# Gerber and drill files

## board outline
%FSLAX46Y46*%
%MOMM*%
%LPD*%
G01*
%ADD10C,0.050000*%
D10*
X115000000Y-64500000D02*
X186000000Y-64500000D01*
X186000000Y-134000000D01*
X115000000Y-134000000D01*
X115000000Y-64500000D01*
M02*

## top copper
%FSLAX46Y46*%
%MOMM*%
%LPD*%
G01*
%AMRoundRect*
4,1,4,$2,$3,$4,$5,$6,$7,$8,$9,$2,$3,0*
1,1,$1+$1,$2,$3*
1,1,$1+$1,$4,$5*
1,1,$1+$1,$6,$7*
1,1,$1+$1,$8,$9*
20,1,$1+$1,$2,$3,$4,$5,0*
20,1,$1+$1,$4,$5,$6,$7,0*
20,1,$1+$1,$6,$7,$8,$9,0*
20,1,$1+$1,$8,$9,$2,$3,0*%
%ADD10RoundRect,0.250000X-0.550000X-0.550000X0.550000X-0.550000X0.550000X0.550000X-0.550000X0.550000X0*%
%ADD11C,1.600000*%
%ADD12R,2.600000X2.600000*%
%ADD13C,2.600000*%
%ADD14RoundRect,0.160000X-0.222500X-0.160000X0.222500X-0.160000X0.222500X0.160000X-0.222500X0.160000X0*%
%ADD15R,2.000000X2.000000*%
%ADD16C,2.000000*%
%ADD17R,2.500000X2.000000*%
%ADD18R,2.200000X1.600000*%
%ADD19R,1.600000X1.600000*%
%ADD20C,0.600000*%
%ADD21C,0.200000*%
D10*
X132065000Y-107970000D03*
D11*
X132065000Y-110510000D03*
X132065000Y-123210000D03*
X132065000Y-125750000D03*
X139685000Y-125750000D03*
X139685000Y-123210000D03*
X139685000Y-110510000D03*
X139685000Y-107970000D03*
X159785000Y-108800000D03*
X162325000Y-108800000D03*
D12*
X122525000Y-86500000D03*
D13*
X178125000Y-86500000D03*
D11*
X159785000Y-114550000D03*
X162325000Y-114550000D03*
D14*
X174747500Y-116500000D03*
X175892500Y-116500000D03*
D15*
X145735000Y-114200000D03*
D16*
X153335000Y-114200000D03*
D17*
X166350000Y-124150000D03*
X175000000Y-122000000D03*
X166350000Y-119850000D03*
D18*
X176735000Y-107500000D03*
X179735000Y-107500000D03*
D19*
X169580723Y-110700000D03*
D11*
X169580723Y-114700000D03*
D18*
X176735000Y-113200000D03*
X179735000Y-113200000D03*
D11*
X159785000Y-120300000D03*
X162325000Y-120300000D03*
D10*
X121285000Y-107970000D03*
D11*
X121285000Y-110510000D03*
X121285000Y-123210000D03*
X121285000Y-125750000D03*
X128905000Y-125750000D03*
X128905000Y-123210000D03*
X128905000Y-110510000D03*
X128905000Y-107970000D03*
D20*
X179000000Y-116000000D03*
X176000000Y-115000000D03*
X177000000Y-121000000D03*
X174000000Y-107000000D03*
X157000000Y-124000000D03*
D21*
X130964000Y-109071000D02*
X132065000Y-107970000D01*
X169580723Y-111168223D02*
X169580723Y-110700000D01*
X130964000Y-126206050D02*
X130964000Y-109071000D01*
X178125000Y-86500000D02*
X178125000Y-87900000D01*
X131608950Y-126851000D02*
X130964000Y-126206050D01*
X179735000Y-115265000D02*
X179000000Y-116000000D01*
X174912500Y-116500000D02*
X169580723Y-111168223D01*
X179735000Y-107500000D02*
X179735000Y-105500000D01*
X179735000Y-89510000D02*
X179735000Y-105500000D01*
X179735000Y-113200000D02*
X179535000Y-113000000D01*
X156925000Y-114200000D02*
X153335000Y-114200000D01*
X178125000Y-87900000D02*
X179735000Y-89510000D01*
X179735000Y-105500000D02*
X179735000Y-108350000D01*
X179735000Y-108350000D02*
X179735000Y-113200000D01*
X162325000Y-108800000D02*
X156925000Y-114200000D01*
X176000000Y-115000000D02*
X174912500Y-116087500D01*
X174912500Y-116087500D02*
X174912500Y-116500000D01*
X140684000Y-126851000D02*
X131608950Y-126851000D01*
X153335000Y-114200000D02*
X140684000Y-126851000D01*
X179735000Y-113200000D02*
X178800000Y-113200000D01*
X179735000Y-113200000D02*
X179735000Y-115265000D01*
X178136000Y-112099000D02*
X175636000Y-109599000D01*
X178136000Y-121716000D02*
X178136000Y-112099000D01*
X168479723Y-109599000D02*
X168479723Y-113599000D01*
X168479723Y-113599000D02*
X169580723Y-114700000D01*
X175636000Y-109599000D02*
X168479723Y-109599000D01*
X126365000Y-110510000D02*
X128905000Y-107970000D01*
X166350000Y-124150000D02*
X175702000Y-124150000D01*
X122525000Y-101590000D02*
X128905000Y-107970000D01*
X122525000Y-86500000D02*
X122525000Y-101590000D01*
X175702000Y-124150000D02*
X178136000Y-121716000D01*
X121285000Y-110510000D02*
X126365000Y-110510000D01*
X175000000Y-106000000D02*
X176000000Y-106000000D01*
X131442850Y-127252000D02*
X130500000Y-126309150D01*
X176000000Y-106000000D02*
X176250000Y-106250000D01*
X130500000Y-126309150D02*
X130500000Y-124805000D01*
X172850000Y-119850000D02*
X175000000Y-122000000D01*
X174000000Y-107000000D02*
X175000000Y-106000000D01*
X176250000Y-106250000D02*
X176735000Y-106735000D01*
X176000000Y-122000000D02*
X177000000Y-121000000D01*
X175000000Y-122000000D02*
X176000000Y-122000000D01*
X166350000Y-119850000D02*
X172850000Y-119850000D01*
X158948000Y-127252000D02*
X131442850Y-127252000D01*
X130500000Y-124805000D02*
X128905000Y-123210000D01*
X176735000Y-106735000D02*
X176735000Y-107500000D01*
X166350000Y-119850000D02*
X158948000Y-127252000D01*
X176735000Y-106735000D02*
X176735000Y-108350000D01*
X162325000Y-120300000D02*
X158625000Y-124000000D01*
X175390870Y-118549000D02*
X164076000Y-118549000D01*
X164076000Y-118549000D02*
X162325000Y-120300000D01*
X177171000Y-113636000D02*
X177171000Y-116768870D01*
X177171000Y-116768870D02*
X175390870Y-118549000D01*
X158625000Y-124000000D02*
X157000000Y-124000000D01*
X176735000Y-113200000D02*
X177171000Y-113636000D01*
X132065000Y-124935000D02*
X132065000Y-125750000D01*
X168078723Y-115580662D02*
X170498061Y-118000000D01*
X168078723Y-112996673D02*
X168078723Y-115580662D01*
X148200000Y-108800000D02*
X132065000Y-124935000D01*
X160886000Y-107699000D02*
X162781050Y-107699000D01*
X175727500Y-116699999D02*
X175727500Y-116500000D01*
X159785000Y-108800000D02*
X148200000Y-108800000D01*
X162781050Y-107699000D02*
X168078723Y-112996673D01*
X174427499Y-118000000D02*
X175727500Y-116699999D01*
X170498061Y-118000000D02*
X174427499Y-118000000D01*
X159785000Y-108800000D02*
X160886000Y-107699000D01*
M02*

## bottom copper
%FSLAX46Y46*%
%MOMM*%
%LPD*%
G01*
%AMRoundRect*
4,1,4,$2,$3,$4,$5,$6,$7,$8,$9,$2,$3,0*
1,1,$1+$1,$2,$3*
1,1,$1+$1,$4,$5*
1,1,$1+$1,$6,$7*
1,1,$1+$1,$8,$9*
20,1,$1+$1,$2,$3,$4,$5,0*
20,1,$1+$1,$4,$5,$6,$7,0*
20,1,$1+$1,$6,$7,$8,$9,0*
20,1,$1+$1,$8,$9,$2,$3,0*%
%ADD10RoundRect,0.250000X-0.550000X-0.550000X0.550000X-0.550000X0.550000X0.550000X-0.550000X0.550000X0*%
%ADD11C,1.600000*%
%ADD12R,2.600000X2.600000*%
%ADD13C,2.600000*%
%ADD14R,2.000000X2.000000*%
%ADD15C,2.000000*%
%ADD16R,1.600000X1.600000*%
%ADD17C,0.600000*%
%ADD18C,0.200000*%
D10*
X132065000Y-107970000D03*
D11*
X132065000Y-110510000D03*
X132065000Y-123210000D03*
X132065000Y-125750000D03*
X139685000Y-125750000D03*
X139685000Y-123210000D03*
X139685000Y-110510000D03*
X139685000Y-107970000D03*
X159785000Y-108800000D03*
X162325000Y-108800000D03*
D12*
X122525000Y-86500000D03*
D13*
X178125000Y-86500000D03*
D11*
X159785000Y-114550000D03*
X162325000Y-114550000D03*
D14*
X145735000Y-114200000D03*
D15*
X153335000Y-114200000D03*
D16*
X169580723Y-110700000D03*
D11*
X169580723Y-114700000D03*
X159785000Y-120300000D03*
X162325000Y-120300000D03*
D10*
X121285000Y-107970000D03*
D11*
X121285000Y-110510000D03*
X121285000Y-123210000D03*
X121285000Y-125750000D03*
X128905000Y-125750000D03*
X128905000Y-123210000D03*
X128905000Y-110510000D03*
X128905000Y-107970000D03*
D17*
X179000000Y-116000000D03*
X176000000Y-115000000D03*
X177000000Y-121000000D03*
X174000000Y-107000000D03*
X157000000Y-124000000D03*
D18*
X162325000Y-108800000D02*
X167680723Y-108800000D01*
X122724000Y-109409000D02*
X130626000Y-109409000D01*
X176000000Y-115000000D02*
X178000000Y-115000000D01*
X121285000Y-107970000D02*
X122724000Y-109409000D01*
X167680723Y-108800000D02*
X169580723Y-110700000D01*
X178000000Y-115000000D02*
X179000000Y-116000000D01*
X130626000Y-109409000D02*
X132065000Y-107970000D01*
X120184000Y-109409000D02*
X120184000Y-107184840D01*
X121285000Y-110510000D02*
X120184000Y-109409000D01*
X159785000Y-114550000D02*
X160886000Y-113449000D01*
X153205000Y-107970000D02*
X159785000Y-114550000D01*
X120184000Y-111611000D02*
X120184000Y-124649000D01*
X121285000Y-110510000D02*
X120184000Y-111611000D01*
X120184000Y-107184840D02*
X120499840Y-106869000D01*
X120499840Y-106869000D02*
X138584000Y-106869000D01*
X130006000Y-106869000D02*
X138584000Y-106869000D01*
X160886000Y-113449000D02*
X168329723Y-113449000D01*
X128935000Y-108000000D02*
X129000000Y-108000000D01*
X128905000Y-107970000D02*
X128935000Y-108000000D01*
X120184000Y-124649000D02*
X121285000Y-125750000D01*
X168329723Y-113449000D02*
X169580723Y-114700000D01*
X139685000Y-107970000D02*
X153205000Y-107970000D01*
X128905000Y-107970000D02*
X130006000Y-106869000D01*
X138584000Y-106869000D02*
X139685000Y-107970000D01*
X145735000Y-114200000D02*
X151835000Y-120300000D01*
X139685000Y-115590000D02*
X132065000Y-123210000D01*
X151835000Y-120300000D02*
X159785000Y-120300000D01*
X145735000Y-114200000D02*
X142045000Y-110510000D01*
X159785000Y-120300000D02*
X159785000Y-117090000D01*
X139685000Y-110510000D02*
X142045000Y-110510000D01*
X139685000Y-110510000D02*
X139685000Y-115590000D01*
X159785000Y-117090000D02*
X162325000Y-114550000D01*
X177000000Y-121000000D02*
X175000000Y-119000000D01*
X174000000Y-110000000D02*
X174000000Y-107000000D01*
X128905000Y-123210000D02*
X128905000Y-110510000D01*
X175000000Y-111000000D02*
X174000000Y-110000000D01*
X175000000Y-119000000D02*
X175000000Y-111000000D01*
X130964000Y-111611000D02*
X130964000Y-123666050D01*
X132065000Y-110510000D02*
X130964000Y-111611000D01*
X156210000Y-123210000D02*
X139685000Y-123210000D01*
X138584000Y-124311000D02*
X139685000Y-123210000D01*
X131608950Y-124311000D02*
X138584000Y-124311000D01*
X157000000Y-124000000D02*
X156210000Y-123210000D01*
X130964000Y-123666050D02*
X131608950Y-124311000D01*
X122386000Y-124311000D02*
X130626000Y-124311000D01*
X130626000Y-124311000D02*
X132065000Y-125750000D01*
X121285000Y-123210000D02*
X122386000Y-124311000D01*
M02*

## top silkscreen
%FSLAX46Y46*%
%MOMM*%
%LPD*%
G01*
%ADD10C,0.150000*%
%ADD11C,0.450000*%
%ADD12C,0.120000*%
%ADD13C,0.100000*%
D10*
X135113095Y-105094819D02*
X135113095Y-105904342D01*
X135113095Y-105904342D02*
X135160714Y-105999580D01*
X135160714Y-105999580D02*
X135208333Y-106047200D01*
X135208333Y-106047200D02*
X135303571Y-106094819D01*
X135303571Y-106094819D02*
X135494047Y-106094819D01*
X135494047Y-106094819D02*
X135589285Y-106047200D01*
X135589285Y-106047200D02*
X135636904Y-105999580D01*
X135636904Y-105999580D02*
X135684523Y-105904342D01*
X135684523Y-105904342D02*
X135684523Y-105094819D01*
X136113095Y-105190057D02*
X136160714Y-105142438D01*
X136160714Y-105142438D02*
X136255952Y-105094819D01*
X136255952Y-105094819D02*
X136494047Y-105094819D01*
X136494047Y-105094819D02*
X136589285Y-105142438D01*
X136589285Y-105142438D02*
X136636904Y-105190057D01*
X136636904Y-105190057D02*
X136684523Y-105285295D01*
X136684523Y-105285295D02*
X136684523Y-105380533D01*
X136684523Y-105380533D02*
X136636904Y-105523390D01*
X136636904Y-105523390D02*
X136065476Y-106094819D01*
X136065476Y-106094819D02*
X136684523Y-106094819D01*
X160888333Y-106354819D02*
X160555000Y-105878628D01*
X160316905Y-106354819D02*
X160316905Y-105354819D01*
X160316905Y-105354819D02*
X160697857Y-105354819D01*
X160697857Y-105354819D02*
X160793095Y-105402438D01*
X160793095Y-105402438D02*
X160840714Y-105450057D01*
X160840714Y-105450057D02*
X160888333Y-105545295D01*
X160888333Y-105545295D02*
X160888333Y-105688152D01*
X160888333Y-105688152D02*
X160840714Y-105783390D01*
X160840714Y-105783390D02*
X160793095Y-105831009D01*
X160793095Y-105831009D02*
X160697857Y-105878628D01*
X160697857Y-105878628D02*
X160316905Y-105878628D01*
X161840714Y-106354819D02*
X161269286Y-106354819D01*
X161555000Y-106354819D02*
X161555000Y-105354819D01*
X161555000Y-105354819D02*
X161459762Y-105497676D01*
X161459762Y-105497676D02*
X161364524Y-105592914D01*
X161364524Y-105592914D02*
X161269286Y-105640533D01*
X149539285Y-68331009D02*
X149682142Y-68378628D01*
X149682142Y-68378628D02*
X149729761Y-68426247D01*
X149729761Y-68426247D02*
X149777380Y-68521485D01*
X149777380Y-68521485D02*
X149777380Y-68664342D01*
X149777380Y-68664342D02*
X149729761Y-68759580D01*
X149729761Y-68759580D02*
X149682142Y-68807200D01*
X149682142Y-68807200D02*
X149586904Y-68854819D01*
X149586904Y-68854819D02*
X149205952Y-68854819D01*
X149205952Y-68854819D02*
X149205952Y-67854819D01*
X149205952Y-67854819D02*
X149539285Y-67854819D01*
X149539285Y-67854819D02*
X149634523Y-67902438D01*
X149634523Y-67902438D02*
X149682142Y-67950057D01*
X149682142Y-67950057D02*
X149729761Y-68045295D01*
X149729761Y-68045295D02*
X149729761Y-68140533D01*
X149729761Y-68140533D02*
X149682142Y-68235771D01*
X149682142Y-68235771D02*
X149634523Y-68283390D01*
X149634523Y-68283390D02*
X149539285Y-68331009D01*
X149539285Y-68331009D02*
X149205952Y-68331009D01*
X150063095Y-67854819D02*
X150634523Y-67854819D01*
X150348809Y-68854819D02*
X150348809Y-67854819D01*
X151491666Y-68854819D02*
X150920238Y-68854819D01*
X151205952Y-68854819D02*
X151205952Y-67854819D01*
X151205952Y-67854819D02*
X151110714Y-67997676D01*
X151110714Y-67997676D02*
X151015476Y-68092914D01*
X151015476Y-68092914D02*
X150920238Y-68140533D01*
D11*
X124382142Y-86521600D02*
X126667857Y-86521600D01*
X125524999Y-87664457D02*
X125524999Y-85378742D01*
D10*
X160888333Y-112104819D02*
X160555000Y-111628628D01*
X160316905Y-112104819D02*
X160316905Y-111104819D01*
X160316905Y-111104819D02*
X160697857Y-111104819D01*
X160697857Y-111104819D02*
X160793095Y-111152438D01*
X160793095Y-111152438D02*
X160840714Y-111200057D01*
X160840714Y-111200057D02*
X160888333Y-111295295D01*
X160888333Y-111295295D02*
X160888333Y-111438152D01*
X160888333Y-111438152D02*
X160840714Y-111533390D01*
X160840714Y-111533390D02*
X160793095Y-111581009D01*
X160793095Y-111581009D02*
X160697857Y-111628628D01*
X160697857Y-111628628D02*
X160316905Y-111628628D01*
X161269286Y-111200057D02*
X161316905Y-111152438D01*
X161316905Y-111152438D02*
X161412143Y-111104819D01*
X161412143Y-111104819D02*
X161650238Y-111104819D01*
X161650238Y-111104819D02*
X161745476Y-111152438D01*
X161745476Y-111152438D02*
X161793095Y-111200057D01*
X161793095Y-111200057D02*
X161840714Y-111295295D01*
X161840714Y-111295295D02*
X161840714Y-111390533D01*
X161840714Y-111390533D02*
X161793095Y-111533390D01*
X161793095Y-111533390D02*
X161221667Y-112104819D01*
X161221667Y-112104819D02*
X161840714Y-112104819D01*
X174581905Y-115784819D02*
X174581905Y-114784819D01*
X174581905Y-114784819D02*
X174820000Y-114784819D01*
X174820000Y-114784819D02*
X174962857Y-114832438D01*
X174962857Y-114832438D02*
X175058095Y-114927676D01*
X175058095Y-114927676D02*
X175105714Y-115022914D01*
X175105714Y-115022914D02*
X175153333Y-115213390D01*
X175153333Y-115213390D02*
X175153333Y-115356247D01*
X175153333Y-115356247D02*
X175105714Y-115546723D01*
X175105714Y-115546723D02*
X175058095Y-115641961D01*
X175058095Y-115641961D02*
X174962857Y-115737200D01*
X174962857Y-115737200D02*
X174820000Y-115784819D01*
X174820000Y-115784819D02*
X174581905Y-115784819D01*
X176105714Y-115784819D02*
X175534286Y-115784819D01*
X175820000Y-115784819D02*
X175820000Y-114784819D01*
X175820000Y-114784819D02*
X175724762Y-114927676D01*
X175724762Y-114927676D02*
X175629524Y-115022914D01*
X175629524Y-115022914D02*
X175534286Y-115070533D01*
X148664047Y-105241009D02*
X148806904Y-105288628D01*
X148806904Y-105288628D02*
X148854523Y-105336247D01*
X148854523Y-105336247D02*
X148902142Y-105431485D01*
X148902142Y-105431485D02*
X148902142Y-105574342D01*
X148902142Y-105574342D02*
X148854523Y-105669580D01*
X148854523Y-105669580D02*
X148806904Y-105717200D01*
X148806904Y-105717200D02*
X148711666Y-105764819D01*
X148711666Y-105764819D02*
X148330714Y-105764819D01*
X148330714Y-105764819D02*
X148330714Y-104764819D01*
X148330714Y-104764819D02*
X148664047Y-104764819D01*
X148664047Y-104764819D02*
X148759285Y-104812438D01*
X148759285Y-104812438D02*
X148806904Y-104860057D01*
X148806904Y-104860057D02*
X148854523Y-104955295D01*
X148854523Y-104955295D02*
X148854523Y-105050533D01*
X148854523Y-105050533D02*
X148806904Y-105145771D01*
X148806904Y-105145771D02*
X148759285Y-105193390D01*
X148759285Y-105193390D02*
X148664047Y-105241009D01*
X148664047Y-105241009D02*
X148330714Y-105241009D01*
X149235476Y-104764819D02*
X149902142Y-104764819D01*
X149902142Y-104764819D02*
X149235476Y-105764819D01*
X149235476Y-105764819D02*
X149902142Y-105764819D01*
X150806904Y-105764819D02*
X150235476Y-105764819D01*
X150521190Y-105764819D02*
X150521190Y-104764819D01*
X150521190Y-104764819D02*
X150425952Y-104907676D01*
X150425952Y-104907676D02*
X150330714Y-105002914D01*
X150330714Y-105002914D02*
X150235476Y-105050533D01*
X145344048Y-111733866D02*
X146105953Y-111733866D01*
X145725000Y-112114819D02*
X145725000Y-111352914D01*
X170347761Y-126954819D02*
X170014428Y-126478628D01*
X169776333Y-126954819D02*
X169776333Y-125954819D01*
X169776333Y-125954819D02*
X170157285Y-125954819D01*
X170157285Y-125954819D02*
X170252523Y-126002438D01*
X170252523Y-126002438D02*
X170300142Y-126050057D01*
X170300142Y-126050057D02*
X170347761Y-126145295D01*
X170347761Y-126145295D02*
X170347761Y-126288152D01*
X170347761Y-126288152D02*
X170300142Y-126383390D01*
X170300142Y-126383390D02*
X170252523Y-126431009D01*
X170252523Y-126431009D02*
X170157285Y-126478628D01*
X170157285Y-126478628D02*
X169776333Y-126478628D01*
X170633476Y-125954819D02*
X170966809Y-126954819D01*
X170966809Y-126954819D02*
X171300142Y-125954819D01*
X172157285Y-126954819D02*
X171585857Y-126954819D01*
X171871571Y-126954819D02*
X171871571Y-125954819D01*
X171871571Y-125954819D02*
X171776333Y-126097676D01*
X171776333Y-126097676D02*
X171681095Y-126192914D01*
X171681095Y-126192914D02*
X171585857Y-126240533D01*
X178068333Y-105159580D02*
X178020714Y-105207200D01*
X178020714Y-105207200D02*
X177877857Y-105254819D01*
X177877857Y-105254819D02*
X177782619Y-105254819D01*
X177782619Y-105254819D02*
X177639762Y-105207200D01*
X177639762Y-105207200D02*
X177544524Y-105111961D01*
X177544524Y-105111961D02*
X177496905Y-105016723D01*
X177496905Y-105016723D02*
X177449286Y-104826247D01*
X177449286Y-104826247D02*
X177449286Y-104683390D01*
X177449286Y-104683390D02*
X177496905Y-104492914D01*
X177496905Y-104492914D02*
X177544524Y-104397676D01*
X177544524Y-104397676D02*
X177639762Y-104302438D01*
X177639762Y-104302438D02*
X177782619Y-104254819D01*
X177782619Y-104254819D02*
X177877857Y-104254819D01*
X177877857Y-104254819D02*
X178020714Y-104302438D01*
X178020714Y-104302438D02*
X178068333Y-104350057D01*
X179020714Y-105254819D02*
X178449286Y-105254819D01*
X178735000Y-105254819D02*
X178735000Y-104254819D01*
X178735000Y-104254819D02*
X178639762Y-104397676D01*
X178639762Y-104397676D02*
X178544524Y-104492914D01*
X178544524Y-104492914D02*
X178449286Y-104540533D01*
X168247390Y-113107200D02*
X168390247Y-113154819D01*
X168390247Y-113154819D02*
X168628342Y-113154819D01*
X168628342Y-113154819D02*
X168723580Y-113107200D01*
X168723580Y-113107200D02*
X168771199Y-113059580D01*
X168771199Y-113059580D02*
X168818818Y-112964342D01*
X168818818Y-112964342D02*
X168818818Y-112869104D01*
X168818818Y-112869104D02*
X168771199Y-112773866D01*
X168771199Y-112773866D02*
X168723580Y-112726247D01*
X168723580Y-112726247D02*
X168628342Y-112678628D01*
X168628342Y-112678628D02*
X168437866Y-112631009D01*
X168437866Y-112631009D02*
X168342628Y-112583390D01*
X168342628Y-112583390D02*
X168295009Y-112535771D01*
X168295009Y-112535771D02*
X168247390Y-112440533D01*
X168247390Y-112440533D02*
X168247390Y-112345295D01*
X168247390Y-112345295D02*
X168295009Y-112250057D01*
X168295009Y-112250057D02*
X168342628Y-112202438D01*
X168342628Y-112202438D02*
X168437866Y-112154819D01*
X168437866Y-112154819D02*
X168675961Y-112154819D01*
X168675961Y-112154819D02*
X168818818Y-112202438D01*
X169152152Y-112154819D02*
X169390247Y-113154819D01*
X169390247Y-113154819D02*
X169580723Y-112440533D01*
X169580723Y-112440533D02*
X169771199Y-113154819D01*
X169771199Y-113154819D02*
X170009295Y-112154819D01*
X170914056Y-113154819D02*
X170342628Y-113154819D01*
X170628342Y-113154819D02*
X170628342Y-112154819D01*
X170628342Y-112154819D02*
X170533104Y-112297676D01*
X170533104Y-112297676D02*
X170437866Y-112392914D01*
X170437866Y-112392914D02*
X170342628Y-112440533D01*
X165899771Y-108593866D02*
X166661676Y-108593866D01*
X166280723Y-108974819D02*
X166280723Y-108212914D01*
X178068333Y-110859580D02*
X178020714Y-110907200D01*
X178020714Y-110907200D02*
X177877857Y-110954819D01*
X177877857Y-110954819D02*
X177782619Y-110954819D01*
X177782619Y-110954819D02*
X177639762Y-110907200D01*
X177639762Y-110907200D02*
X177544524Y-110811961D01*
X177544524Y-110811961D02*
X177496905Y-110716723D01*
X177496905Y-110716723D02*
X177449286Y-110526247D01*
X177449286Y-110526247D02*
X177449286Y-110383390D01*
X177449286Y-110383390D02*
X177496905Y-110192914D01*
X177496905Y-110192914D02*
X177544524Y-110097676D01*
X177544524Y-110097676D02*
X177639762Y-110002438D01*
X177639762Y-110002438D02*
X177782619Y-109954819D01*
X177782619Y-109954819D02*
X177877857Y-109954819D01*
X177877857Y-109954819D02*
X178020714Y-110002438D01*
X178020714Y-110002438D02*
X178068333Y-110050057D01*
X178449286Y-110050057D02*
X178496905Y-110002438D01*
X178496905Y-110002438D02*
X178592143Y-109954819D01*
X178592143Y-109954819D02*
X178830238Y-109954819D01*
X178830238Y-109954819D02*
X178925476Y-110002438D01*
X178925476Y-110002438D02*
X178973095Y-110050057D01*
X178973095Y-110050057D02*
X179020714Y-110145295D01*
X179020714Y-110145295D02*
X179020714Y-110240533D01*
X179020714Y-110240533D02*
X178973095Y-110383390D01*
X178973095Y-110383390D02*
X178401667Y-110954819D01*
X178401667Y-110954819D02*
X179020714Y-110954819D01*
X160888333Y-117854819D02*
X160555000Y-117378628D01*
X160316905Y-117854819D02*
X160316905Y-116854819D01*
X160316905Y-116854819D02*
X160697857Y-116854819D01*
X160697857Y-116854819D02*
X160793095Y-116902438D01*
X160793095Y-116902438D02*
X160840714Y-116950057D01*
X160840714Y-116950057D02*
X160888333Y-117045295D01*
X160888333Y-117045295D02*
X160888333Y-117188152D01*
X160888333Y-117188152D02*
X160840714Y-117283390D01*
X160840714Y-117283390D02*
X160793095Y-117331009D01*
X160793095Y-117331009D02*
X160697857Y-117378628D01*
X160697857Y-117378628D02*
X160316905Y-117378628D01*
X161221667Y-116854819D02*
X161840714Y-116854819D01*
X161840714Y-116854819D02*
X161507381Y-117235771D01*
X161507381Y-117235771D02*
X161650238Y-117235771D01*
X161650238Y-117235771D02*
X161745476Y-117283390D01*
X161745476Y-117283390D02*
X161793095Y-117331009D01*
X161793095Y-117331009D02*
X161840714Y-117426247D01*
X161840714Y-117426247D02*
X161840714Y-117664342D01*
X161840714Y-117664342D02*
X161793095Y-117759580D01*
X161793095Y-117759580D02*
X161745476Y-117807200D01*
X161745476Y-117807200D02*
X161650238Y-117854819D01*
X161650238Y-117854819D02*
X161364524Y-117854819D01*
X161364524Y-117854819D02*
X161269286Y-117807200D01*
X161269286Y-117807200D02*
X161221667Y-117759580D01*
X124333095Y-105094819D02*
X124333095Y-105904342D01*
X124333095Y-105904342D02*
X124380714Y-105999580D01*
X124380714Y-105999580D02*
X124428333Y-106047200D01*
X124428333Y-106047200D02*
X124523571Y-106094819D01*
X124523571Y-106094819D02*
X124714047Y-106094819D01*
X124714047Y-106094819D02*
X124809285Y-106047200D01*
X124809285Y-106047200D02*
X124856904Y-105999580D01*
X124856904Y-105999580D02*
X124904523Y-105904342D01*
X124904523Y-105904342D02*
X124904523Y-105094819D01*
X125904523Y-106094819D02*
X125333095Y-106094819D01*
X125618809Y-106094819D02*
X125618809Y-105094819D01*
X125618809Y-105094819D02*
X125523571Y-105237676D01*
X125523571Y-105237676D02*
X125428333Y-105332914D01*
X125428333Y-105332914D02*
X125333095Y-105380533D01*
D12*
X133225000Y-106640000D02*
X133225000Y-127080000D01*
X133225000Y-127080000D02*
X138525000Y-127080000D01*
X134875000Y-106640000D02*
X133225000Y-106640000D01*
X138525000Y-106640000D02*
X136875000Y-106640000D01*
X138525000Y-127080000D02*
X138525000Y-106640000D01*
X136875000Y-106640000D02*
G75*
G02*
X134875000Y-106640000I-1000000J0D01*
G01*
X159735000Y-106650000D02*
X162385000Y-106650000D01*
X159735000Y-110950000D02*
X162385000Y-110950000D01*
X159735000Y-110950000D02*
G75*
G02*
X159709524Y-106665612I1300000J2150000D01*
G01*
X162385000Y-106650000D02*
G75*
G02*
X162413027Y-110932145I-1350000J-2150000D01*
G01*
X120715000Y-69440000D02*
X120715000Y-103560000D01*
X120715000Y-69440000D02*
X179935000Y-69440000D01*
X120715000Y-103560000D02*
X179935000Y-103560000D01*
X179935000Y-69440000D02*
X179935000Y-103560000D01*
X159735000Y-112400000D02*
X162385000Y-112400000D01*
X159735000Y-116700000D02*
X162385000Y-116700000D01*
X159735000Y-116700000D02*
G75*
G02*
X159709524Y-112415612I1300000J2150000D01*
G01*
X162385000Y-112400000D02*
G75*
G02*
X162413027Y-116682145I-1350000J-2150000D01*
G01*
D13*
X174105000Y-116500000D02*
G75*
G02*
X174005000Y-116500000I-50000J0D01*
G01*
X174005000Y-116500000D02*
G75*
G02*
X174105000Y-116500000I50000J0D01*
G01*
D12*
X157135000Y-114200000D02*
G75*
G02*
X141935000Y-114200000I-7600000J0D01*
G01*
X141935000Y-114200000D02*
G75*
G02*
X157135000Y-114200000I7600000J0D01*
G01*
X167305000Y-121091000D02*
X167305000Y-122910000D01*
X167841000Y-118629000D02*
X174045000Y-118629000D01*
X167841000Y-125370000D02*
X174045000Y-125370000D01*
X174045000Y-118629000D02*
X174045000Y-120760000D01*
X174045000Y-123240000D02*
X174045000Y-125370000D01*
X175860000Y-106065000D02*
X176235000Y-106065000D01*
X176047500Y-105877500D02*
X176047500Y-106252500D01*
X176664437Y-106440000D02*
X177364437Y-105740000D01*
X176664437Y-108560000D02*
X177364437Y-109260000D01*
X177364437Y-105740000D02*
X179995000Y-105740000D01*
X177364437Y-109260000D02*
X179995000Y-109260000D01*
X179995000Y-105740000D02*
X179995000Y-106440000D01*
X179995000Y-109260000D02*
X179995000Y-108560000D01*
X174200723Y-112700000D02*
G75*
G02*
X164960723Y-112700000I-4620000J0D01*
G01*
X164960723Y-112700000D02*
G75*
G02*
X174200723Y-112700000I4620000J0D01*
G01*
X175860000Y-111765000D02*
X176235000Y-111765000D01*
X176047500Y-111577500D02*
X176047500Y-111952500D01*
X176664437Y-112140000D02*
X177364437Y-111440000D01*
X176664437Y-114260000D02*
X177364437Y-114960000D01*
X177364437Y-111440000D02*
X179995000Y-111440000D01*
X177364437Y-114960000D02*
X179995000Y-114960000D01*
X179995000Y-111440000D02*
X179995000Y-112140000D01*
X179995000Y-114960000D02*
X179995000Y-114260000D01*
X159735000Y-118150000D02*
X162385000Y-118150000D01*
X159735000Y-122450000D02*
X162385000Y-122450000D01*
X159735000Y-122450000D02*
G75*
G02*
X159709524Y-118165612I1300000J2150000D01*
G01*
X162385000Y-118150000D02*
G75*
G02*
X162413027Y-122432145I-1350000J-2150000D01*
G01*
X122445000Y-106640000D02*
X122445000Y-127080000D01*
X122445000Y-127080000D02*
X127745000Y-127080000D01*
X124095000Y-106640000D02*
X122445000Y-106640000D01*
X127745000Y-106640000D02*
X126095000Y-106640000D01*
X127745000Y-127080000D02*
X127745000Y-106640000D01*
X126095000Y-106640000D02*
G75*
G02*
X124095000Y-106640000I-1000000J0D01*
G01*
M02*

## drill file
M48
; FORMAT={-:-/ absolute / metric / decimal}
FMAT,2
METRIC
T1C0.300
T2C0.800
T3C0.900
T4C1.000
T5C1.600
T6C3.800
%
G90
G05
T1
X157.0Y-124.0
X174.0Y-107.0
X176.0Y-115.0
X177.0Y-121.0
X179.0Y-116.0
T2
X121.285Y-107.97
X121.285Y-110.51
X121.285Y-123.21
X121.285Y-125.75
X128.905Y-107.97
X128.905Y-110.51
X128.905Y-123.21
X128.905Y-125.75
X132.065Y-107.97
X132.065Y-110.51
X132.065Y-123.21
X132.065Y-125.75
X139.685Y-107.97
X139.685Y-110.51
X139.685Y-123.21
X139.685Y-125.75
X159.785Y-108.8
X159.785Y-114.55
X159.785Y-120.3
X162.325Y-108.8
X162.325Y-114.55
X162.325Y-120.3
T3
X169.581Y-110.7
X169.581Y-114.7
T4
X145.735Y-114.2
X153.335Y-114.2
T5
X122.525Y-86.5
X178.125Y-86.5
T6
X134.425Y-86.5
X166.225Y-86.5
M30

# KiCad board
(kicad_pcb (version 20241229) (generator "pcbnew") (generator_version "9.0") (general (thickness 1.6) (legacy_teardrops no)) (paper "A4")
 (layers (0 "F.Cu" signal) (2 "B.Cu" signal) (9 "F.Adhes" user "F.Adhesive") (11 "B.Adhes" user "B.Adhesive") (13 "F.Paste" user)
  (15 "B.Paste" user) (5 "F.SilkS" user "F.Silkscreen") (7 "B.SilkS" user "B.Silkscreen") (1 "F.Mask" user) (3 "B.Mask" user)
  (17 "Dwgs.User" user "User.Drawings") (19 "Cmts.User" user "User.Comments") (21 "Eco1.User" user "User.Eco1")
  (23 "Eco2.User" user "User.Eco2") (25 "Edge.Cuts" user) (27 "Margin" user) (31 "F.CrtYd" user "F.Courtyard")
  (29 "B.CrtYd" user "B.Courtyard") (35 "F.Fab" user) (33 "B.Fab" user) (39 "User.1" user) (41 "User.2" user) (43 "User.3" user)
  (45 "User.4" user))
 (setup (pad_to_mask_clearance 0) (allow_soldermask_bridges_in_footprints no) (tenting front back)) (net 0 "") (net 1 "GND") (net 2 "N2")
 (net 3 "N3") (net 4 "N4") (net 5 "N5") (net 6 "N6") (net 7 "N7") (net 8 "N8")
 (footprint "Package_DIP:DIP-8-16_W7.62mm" (layer "F.Cu") (at 132.065 107.97)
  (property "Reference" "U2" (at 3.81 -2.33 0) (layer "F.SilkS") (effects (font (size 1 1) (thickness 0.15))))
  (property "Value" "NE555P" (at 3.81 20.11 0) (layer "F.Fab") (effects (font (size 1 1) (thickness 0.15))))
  (fp_line (start 1.16 -1.33) (end 1.16 19.11) (stroke (width 0.12) (type solid)) (layer "F.SilkS"))
  (fp_line (start 1.16 19.11) (end 6.46 19.11) (stroke (width 0.12) (type solid)) (layer "F.SilkS"))
  (fp_line (start 2.81 -1.33) (end 1.16 -1.33) (stroke (width 0.12) (type solid)) (layer "F.SilkS"))
  (fp_line (start 6.46 -1.33) (end 4.81 -1.33) (stroke (width 0.12) (type solid)) (layer "F.SilkS"))
  (fp_line (start 6.46 19.11) (end 6.46 -1.33) (stroke (width 0.12) (type solid)) (layer "F.SilkS"))
  (fp_arc (start 4.81 -1.33) (mid 3.81 -0.33) (end 2.81 -1.33) (stroke (width 0.12) (type solid)) (layer "F.SilkS"))
  (pad "1" thru_hole roundrect (at 0 0) (size 1.6 1.6) (drill 0.8) (layers "*.Cu" "*.Mask") (remove_unused_layers no)
   (roundrect_rratio 0.15625) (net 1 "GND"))
  (pad "2" thru_hole circle (at 0 2.54) (size 1.6 1.6) (drill 0.8) (layers "*.Cu" "*.Mask") (remove_unused_layers no) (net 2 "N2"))
  (pad "3" thru_hole circle (at 0 15.24) (size 1.6 1.6) (drill 0.8) (layers "*.Cu" "*.Mask") (remove_unused_layers no) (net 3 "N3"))
  (pad "4" thru_hole circle (at 0 17.78) (size 1.6 1.6) (drill 0.8) (layers "*.Cu" "*.Mask") (remove_unused_layers no) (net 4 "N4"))
  (pad "5" thru_hole circle (at 7.62 17.78) (size 1.6 1.6) (drill 0.8) (layers "*.Cu" "*.Mask") (remove_unused_layers no) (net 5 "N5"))
  (pad "6" thru_hole circle (at 7.62 15.24) (size 1.6 1.6) (drill 0.8) (layers "*.Cu" "*.Mask") (remove_unused_layers no) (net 2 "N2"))
  (pad "7" thru_hole circle (at 7.62 2.54) (size 1.6 1.6) (drill 0.8) (layers "*.Cu" "*.Mask") (remove_unused_layers no) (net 3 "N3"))
  (pad "8" thru_hole circle (at 7.62 0) (size 1.6 1.6) (drill 0.8) (layers "*.Cu" "*.Mask") (remove_unused_layers no) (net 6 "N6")))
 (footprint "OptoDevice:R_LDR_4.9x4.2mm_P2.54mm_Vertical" (layer "F.Cu") (at 159.785 108.8)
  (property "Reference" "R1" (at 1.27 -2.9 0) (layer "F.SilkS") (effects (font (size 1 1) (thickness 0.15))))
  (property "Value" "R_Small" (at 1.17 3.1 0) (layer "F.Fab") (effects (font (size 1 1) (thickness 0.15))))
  (fp_line (start -0.05 -2.15) (end 2.6 -2.15) (stroke (width 0.12) (type solid)) (layer "F.SilkS"))
  (fp_line (start -0.05 2.15) (end 2.6 2.15) (stroke (width 0.12) (type solid)) (layer "F.SilkS"))
  (fp_arc (start -0.05 2.15) (mid -1.262424 0.01494) (end -0.075476 -2.134388) (stroke (width 0.12) (type solid)) (layer "F.SilkS"))
  (fp_arc (start 2.6 -2.15) (mid 3.788646 -0.016616) (end 2.628027 2.132145) (stroke (width 0.12) (type solid)) (layer "F.SilkS"))
  (pad "1" thru_hole circle (at 0 0) (size 1.6 1.6) (drill 0.8) (layers "*.Cu" "*.Mask") (remove_unused_layers no) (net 4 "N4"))
  (pad "2" thru_hole circle (at 2.54 0) (size 1.6 1.6) (drill 0.8) (layers "*.Cu" "*.Mask") (remove_unused_layers no) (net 1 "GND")))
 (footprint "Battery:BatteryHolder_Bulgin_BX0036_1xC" (layer "F.Cu") (at 122.525 86.5)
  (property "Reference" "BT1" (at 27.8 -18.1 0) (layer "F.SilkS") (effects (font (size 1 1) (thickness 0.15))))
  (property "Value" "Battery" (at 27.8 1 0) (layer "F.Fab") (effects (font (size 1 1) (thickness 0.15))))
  (fp_line (start -1.81 -17.06) (end -1.81 17.06) (stroke (width 0.12) (type solid)) (layer "F.SilkS"))
  (fp_line (start -1.81 -17.06) (end 57.41 -17.06) (stroke (width 0.12) (type solid)) (layer "F.SilkS"))
  (fp_line (start -1.81 17.06) (end 57.41 17.06) (stroke (width 0.12) (type solid)) (layer "F.SilkS"))
  (fp_line (start 57.41 -17.06) (end 57.41 17.06) (stroke (width 0.12) (type solid)) (layer "F.SilkS"))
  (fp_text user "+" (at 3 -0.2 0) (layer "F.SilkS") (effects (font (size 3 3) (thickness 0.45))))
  (pad "" np_thru_hole circle (at 11.9 0) (size 3.8 3.8) (drill 3.8) (layers "*.Cu" "*.Mask"))
  (pad "" np_thru_hole circle (at 43.7 0) (size 3.8 3.8) (drill 3.8) (layers "*.Cu" "*.Mask"))
  (pad "1" thru_hole rect (at 0 0) (size 2.6 2.6) (drill 1.6) (layers "*.Cu" "*.Mask") (remove_unused_layers no) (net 6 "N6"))
  (pad "2" thru_hole circle (at 55.6 0) (size 2.6 2.6) (drill 1.6) (layers "*.Cu" "*.Mask") (remove_unused_layers no) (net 1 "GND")))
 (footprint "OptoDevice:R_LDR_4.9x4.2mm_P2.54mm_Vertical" (layer "F.Cu") (at 159.785 114.55)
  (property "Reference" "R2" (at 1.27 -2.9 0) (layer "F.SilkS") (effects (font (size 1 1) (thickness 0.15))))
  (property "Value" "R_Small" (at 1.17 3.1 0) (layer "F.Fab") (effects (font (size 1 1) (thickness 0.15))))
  (fp_line (start -0.05 -2.15) (end 2.6 -2.15) (stroke (width 0.12) (type solid)) (layer "F.SilkS"))
  (fp_line (start -0.05 2.15) (end 2.6 2.15) (stroke (width 0.12) (type solid)) (layer "F.SilkS"))
  (fp_arc (start -0.05 2.15) (mid -1.262424 0.01494) (end -0.075476 -2.134388) (stroke (width 0.12) (type solid)) (layer "F.SilkS"))
  (fp_arc (start 2.6 -2.15) (mid 3.788646 -0.016616) (end 2.628027 2.132145) (stroke (width 0.12) (type solid)) (layer "F.SilkS"))
  (pad "1" thru_hole circle (at 0 0) (size 1.6 1.6) (drill 0.8) (layers "*.Cu" "*.Mask") (remove_unused_layers no) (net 6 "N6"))
  (pad "2" thru_hole circle (at 2.54 0) (size 1.6 1.6) (drill 0.8) (layers "*.Cu" "*.Mask") (remove_unused_layers no) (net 3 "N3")))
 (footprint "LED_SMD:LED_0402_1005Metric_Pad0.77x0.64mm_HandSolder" (layer "F.Cu") (at 175.32 116.5)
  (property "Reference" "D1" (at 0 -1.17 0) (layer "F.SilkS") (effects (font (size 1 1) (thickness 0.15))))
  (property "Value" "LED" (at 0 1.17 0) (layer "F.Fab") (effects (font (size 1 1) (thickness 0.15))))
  (fp_circle (center -1.265 0) (end -1.215 0) (stroke (width 0.1) (type solid)) (fill no) (layer "F.SilkS"))
  (pad "1" smd roundrect (at -0.5725 0) (size 0.765 0.64) (layers "F.Cu" "F.Mask" "F.Paste") (roundrect_rratio 0.25) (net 1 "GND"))
  (pad "2" smd roundrect (at 0.5725 0) (size 0.765 0.64) (layers "F.Cu" "F.Mask" "F.Paste") (roundrect_rratio 0.25) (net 4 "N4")))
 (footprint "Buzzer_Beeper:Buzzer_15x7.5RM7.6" (layer "F.Cu") (at 145.735 114.2)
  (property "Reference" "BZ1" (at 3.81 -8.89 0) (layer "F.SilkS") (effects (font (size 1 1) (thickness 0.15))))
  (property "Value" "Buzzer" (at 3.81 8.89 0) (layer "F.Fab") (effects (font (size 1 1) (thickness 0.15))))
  (fp_circle (center 3.8 0) (end 11.4 0) (stroke (width 0.12) (type solid)) (fill no) (layer "F.SilkS"))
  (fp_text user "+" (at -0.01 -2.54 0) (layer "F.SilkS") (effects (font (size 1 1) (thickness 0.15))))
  (pad "1" thru_hole rect (at 0 0) (size 2 2) (drill 1) (layers "*.Cu" "*.Mask") (remove_unused_layers no) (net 3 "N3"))
  (pad "2" thru_hole circle (at 7.6 0) (size 2 2) (drill 1) (layers "*.Cu" "*.Mask") (remove_unused_layers no) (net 1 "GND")))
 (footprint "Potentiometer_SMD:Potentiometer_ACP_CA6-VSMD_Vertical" (layer "F.Cu") (at 170.675 122)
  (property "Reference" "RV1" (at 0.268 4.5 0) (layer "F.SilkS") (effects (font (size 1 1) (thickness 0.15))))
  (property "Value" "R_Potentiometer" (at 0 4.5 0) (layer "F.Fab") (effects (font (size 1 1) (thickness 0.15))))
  (fp_line (start -3.37 -0.909) (end -3.37 0.91) (stroke (width 0.12) (type solid)) (layer "F.SilkS"))
  (fp_line (start -2.834 -3.371) (end 3.37 -3.371) (stroke (width 0.12) (type solid)) (layer "F.SilkS"))
  (fp_line (start -2.834 3.37) (end 3.37 3.37) (stroke (width 0.12) (type solid)) (layer "F.SilkS"))
  (fp_line (start 3.37 -3.371) (end 3.37 -1.24) (stroke (width 0.12) (type solid)) (layer "F.SilkS"))
  (fp_line (start 3.37 1.24) (end 3.37 3.37) (stroke (width 0.12) (type solid)) (layer "F.SilkS"))
  (pad "1" smd rect (at -4.325 2.15) (size 2.5 2) (layers "F.Cu" "F.Mask" "F.Paste") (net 6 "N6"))
  (pad "2" smd rect (at 4.325 0) (size 2.5 2) (layers "F.Cu" "F.Mask" "F.Paste") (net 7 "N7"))
  (pad "3" smd rect (at -4.325 -2.15) (size 2.5 2) (layers "F.Cu" "F.Mask" "F.Paste") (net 7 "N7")))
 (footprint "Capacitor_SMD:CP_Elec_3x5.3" (layer "F.Cu") (at 178.235 107.5)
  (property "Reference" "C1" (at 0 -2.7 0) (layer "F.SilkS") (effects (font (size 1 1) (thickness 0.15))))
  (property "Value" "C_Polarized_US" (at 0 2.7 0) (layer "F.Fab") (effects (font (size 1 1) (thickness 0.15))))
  (fp_line (start -2.375 -1.435) (end -2 -1.435) (stroke (width 0.12) (type solid)) (layer "F.SilkS"))
  (fp_line (start -2.1875 -1.6225) (end -2.1875 -1.2475) (stroke (width 0.12) (type solid)) (layer "F.SilkS"))
  (fp_line (start -1.570563 -1.06) (end -0.870563 -1.76) (stroke (width 0.12) (type solid)) (layer "F.SilkS"))
  (fp_line (start -1.570563 1.06) (end -0.870563 1.76) (stroke (width 0.12) (type solid)) (layer "F.SilkS"))
  (fp_line (start -0.870563 -1.76) (end 1.76 -1.76) (stroke (width 0.12) (type solid)) (layer "F.SilkS"))
  (fp_line (start -0.870563 1.76) (end 1.76 1.76) (stroke (width 0.12) (type solid)) (layer "F.SilkS"))
  (fp_line (start 1.76 -1.76) (end 1.76 -1.06) (stroke (width 0.12) (type solid)) (layer "F.SilkS"))
  (fp_line (start 1.76 1.76) (end 1.76 1.06) (stroke (width 0.12) (type solid)) (layer "F.SilkS"))
  (pad "1" smd rect (at -1.5 0) (size 2.2 1.6) (layers "F.Cu" "F.Mask" "F.Paste") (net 7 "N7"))
  (pad "2" smd rect (at 1.5 0) (size 2.2 1.6) (layers "F.Cu" "F.Mask" "F.Paste") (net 1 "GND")))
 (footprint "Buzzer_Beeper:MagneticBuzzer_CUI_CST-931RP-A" (layer "F.Cu") (at 169.580723 110.7)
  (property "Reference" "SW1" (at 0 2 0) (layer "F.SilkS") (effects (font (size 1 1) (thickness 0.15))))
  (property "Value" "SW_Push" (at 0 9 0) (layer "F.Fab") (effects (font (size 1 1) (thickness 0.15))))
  (fp_circle (center 0 2) (end 4.62 2) (stroke (width 0.12) (type solid)) (fill no) (layer "F.SilkS"))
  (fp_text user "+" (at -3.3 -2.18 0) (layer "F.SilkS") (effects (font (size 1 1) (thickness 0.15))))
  (pad "1" thru_hole rect (at 0 0) (size 1.6 1.6) (drill 0.9) (layers "*.Cu" "*.Mask") (remove_unused_layers no) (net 1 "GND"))
  (pad "2" thru_hole circle (at 0 4) (size 1.6 1.6) (drill 0.9) (layers "*.Cu" "*.Mask") (remove_unused_layers no) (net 6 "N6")))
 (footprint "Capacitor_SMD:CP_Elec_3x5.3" (layer "F.Cu") (at 178.235 113.2)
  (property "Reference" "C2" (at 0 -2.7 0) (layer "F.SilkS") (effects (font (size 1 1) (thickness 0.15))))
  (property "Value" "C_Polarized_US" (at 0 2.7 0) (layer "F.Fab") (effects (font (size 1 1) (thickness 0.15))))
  (fp_line (start -2.375 -1.435) (end -2 -1.435) (stroke (width 0.12) (type solid)) (layer "F.SilkS"))
  (fp_line (start -2.1875 -1.6225) (end -2.1875 -1.2475) (stroke (width 0.12) (type solid)) (layer "F.SilkS"))
  (fp_line (start -1.570563 -1.06) (end -0.870563 -1.76) (stroke (width 0.12) (type solid)) (layer "F.SilkS"))
  (fp_line (start -1.570563 1.06) (end -0.870563 1.76) (stroke (width 0.12) (type solid)) (layer "F.SilkS"))
  (fp_line (start -0.870563 -1.76) (end 1.76 -1.76) (stroke (width 0.12) (type solid)) (layer "F.SilkS"))
  (fp_line (start -0.870563 1.76) (end 1.76 1.76) (stroke (width 0.12) (type solid)) (layer "F.SilkS"))
  (fp_line (start 1.76 -1.76) (end 1.76 -1.06) (stroke (width 0.12) (type solid)) (layer "F.SilkS"))
  (fp_line (start 1.76 1.76) (end 1.76 1.06) (stroke (width 0.12) (type solid)) (layer "F.SilkS"))
  (pad "1" smd rect (at -1.5 0) (size 2.2 1.6) (layers "F.Cu" "F.Mask" "F.Paste") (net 2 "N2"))
  (pad "2" smd rect (at 1.5 0) (size 2.2 1.6) (layers "F.Cu" "F.Mask" "F.Paste") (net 1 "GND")))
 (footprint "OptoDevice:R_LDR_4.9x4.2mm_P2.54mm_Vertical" (layer "F.Cu") (at 159.785 120.3)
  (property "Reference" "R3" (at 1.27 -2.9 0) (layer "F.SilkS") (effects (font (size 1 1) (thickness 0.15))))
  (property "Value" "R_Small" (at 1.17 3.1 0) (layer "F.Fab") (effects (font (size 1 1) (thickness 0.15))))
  (fp_line (start -0.05 -2.15) (end 2.6 -2.15) (stroke (width 0.12) (type solid)) (layer "F.SilkS"))
  (fp_line (start -0.05 2.15) (end 2.6 2.15) (stroke (width 0.12) (type solid)) (layer "F.SilkS"))
  (fp_arc (start -0.05 2.15) (mid -1.262424 0.01494) (end -0.075476 -2.134388) (stroke (width 0.12) (type solid)) (layer "F.SilkS"))
  (fp_arc (start 2.6 -2.15) (mid 3.788646 -0.016616) (end 2.628027 2.132145) (stroke (width 0.12) (type solid)) (layer "F.SilkS"))
  (pad "1" thru_hole circle (at 0 0) (size 1.6 1.6) (drill 0.8) (layers "*.Cu" "*.Mask") (remove_unused_layers no) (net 3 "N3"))
  (pad "2" thru_hole circle (at 2.54 0) (size 1.6 1.6) (drill 0.8) (layers "*.Cu" "*.Mask") (remove_unused_layers no) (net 2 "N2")))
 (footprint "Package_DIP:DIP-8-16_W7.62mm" (layer "F.Cu") (at 121.285 107.97)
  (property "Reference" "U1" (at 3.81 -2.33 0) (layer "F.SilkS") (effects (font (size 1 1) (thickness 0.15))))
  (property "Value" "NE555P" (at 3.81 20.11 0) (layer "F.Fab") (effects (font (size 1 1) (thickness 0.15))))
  (fp_line (start 1.16 -1.33) (end 1.16 19.11) (stroke (width 0.12) (type solid)) (layer "F.SilkS"))
  (fp_line (start 1.16 19.11) (end 6.46 19.11) (stroke (width 0.12) (type solid)) (layer "F.SilkS"))
  (fp_line (start 2.81 -1.33) (end 1.16 -1.33) (stroke (width 0.12) (type solid)) (layer "F.SilkS"))
  (fp_line (start 6.46 -1.33) (end 4.81 -1.33) (stroke (width 0.12) (type solid)) (layer "F.SilkS"))
  (fp_line (start 6.46 19.11) (end 6.46 -1.33) (stroke (width 0.12) (type solid)) (layer "F.SilkS"))
  (fp_arc (start 4.81 -1.33) (mid 3.81 -0.33) (end 2.81 -1.33) (stroke (width 0.12) (type solid)) (layer "F.SilkS"))
  (pad "1" thru_hole roundrect (at 0 0) (size 1.6 1.6) (drill 0.8) (layers "*.Cu" "*.Mask") (remove_unused_layers no)
   (roundrect_rratio 0.15625) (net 1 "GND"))
  (pad "2" thru_hole circle (at 0 2.54) (size 1.6 1.6) (drill 0.8) (layers "*.Cu" "*.Mask") (remove_unused_layers no) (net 6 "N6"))
  (pad "3" thru_hole circle (at 0 15.24) (size 1.6 1.6) (drill 0.8) (layers "*.Cu" "*.Mask") (remove_unused_layers no) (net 4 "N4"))
  (pad "4" thru_hole circle (at 0 17.78) (size 1.6 1.6) (drill 0.8) (layers "*.Cu" "*.Mask") (remove_unused_layers no) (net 6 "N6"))
  (pad "5" thru_hole circle (at 7.62 17.78) (size 1.6 1.6) (drill 0.8) (layers "*.Cu" "*.Mask") (remove_unused_layers no) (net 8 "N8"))
  (pad "6" thru_hole circle (at 7.62 15.24) (size 1.6 1.6) (drill 0.8) (layers "*.Cu" "*.Mask") (remove_unused_layers no) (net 7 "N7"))
  (pad "7" thru_hole circle (at 7.62 2.54) (size 1.6 1.6) (drill 0.8) (layers "*.Cu" "*.Mask") (remove_unused_layers no) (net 7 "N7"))
  (pad "8" thru_hole circle (at 7.62 0) (size 1.6 1.6) (drill 0.8) (layers "*.Cu" "*.Mask") (remove_unused_layers no) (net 6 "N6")))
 (gr_rect (start 115 64.5) (end 186 134) (stroke (width 0.05) (type default)) (fill no) (layer "Edge.Cuts"))
 (segment (start 130.964 109.071) (end 132.065 107.97) (width 0.2) (layer "F.Cu") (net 1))
 (segment (start 169.580723 111.168223) (end 169.580723 110.7) (width 0.2) (layer "F.Cu") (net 1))
 (segment (start 130.964 126.20605) (end 130.964 109.071) (width 0.2) (layer "F.Cu") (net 1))
 (segment (start 178.125 86.5) (end 178.125 87.9) (width 0.2) (layer "F.Cu") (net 1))
 (segment (start 131.60895 126.851) (end 130.964 126.20605) (width 0.2) (layer "F.Cu") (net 1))
 (segment (start 179.735 115.265) (end 179 116) (width 0.2) (layer "F.Cu") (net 1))
 (segment (start 174.9125 116.5) (end 169.580723 111.168223) (width 0.2) (layer "F.Cu") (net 1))
 (segment (start 179.735 107.5) (end 179.735 105.5) (width 0.2) (layer "F.Cu") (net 1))
 (segment (start 179.735 89.51) (end 179.735 105.5) (width 0.2) (layer "F.Cu") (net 1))
 (segment (start 179.735 113.2) (end 179.535 113) (width 0.2) (layer "F.Cu") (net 1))
 (segment (start 156.925 114.2) (end 153.335 114.2) (width 0.2) (layer "F.Cu") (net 1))
 (segment (start 178.125 87.9) (end 179.735 89.51) (width 0.2) (layer "F.Cu") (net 1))
 (segment (start 179.735 105.5) (end 179.735 108.35) (width 0.2) (layer "F.Cu") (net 1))
 (segment (start 179.735 108.35) (end 179.735 113.2) (width 0.2) (layer "F.Cu") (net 1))
 (segment (start 162.325 108.8) (end 156.925 114.2) (width 0.2) (layer "F.Cu") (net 1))
 (segment (start 176 115) (end 174.9125 116.0875) (width 0.2) (layer "F.Cu") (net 1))
 (segment (start 174.9125 116.0875) (end 174.9125 116.5) (width 0.2) (layer "F.Cu") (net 1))
 (segment (start 140.684 126.851) (end 131.60895 126.851) (width 0.2) (layer "F.Cu") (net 1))
 (segment (start 153.335 114.2) (end 140.684 126.851) (width 0.2) (layer "F.Cu") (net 1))
 (segment (start 179.735 113.2) (end 178.8 113.2) (width 0.2) (layer "F.Cu") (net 1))
 (segment (start 179.735 113.2) (end 179.735 115.265) (width 0.2) (layer "F.Cu") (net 1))
 (via (at 179 116) (size 0.6) (drill 0.3) (layers "F.Cu" "B.Cu") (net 1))
 (via (at 176 115) (size 0.6) (drill 0.3) (layers "F.Cu" "B.Cu") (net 1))
 (segment (start 162.325 108.8) (end 167.680723 108.8) (width 0.2) (layer "B.Cu") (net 1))
 (segment (start 122.724 109.409) (end 130.626 109.409) (width 0.2) (layer "B.Cu") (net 1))
 (segment (start 176 115) (end 178 115) (width 0.2) (layer "B.Cu") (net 1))
 (segment (start 121.285 107.97) (end 122.724 109.409) (width 0.2) (layer "B.Cu") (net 1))
 (segment (start 167.680723 108.8) (end 169.580723 110.7) (width 0.2) (layer "B.Cu") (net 1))
 (segment (start 178 115) (end 179 116) (width 0.2) (layer "B.Cu") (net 1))
 (segment (start 130.626 109.409) (end 132.065 107.97) (width 0.2) (layer "B.Cu") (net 1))
 (segment (start 178.136 112.099) (end 175.636 109.599) (width 0.2) (layer "F.Cu") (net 6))
 (segment (start 178.136 121.716) (end 178.136 112.099) (width 0.2) (layer "F.Cu") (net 6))
 (segment (start 168.479723 109.599) (end 168.479723 113.599) (width 0.2) (layer "F.Cu") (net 6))
 (segment (start 168.479723 113.599) (end 169.580723 114.7) (width 0.2) (layer "F.Cu") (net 6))
 (segment (start 175.636 109.599) (end 168.479723 109.599) (width 0.2) (layer "F.Cu") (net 6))
 (segment (start 126.365 110.51) (end 128.905 107.97) (width 0.2) (layer "F.Cu") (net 6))
 (segment (start 166.35 124.15) (end 175.702 124.15) (width 0.2) (layer "F.Cu") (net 6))
 (segment (start 122.525 101.59) (end 128.905 107.97) (width 0.2) (layer "F.Cu") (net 6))
 (segment (start 122.525 86.5) (end 122.525 101.59) (width 0.2) (layer "F.Cu") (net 6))
 (segment (start 175.702 124.15) (end 178.136 121.716) (width 0.2) (layer "F.Cu") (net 6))
 (segment (start 121.285 110.51) (end 126.365 110.51) (width 0.2) (layer "F.Cu") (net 6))
 (segment (start 120.184 109.409) (end 120.184 107.18484) (width 0.2) (layer "B.Cu") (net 6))
 (segment (start 121.285 110.51) (end 120.184 109.409) (width 0.2) (layer "B.Cu") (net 6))
 (segment (start 159.785 114.55) (end 160.886 113.449) (width 0.2) (layer "B.Cu") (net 6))
 (segment (start 153.205 107.97) (end 159.785 114.55) (width 0.2) (layer "B.Cu") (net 6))
 (segment (start 120.184 111.611) (end 120.184 124.649) (width 0.2) (layer "B.Cu") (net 6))
 (segment (start 121.285 110.51) (end 120.184 111.611) (width 0.2) (layer "B.Cu") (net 6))
 (segment (start 120.184 107.18484) (end 120.49984 106.869) (width 0.2) (layer "B.Cu") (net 6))
 (segment (start 120.49984 106.869) (end 138.584 106.869) (width 0.2) (layer "B.Cu") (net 6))
 (segment (start 130.006 106.869) (end 138.584 106.869) (width 0.2) (layer "B.Cu") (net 6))
 (segment (start 160.886 113.449) (end 168.329723 113.449) (width 0.2) (layer "B.Cu") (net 6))
 (segment (start 128.935 108) (end 129 108) (width 0.2) (layer "B.Cu") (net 6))
 (segment (start 128.905 107.97) (end 128.935 108) (width 0.2) (layer "B.Cu") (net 6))
 (segment (start 120.184 124.649) (end 121.285 125.75) (width 0.2) (layer "B.Cu") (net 6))
 (segment (start 168.329723 113.449) (end 169.580723 114.7) (width 0.2) (layer "B.Cu") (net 6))
 (segment (start 139.685 107.97) (end 153.205 107.97) (width 0.2) (layer "B.Cu") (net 6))
 (segment (start 128.905 107.97) (end 130.006 106.869) (width 0.2) (layer "B.Cu") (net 6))
 (segment (start 138.584 106.869) (end 139.685 107.97) (width 0.2) (layer "B.Cu") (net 6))
 (segment (start 145.735 114.2) (end 151.835 120.3) (width 0.2) (layer "B.Cu") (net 3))
 (segment (start 139.685 115.59) (end 132.065 123.21) (width 0.2) (layer "B.Cu") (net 3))
 (segment (start 151.835 120.3) (end 159.785 120.3) (width 0.2) (layer "B.Cu") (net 3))
 (segment (start 145.735 114.2) (end 142.045 110.51) (width 0.2) (layer "B.Cu") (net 3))
 (segment (start 159.785 120.3) (end 159.785 117.09) (width 0.2) (layer "B.Cu") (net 3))
 (segment (start 139.685 110.51) (end 142.045 110.51) (width 0.2) (layer "B.Cu") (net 3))
 (segment (start 139.685 110.51) (end 139.685 115.59) (width 0.2) (layer "B.Cu") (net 3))
 (segment (start 159.785 117.09) (end 162.325 114.55) (width 0.2) (layer "B.Cu") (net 3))
 (segment (start 175 106) (end 176 106) (width 0.2) (layer "F.Cu") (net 7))
 (segment (start 131.44285 127.252) (end 130.5 126.30915) (width 0.2) (layer "F.Cu") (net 7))
 (segment (start 176 106) (end 176.25 106.25) (width 0.2) (layer "F.Cu") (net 7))
 (segment (start 130.5 126.30915) (end 130.5 124.805) (width 0.2) (layer "F.Cu") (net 7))
 (segment (start 172.85 119.85) (end 175 122) (width 0.2) (layer "F.Cu") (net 7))
 (segment (start 174 107) (end 175 106) (width 0.2) (layer "F.Cu") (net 7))
 (segment (start 176.25 106.25) (end 176.735 106.735) (width 0.2) (layer "F.Cu") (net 7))
 (segment (start 176 122) (end 177 121) (width 0.2) (layer "F.Cu") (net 7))
 (segment (start 175 122) (end 176 122) (width 0.2) (layer "F.Cu") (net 7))
 (segment (start 166.35 119.85) (end 172.85 119.85) (width 0.2) (layer "F.Cu") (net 7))
 (segment (start 158.948 127.252) (end 131.44285 127.252) (width 0.2) (layer "F.Cu") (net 7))
 (segment (start 130.5 124.805) (end 128.905 123.21) (width 0.2) (layer "F.Cu") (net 7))
 (segment (start 176.735 106.735) (end 176.735 107.5) (width 0.2) (layer "F.Cu") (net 7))
 (segment (start 166.35 119.85) (end 158.948 127.252) (width 0.2) (layer "F.Cu") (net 7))
 (segment (start 176.735 106.735) (end 176.735 108.35) (width 0.2) (layer "F.Cu") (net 7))
 (via (at 177 121) (size 0.6) (drill 0.3) (layers "F.Cu" "B.Cu") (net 7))
 (via (at 174 107) (size 0.6) (drill 0.3) (layers "F.Cu" "B.Cu") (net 7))
 (segment (start 177 121) (end 175 119) (width 0.2) (layer "B.Cu") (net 7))
 (segment (start 174 110) (end 174 107) (width 0.2) (layer "B.Cu") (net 7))
 (segment (start 128.905 123.21) (end 128.905 110.51) (width 0.2) (layer "B.Cu") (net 7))
 (segment (start 175 111) (end 174 110) (width 0.2) (layer "B.Cu") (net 7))
 (segment (start 175 119) (end 175 111) (width 0.2) (layer "B.Cu") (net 7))
 (segment (start 162.325 120.3) (end 158.625 124) (width 0.2) (layer "F.Cu") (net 2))
 (segment (start 175.39087 118.549) (end 164.076 118.549) (width 0.2) (layer "F.Cu") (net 2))
 (segment (start 164.076 118.549) (end 162.325 120.3) (width 0.2) (layer "F.Cu") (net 2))
 (segment (start 177.171 113.636) (end 177.171 116.76887) (width 0.2) (layer "F.Cu") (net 2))
 (segment (start 177.171 116.76887) (end 175.39087 118.549) (width 0.2) (layer "F.Cu") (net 2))
 (segment (start 158.625 124) (end 157 124) (width 0.2) (layer "F.Cu") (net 2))
 (segment (start 176.735 113.2) (end 177.171 113.636) (width 0.2) (layer "F.Cu") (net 2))
 (via (at 157 124) (size 0.6) (drill 0.3) (layers "F.Cu" "B.Cu") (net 2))
 (segment (start 130.964 111.611) (end 130.964 123.66605) (width 0.2) (layer "B.Cu") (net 2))
 (segment (start 132.065 110.51) (end 130.964 111.611) (width 0.2) (layer "B.Cu") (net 2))
 (segment (start 156.21 123.21) (end 139.685 123.21) (width 0.2) (layer "B.Cu") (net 2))
 (segment (start 138.584 124.311) (end 139.685 123.21) (width 0.2) (layer "B.Cu") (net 2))
 (segment (start 131.60895 124.311) (end 138.584 124.311) (width 0.2) (layer "B.Cu") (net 2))
 (segment (start 157 124) (end 156.21 123.21) (width 0.2) (layer "B.Cu") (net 2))
 (segment (start 130.964 123.66605) (end 131.60895 124.311) (width 0.2) (layer "B.Cu") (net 2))
 (segment (start 132.065 124.935) (end 132.065 125.75) (width 0.2) (layer "F.Cu") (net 4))
 (segment (start 168.078723 115.580662) (end 170.498061 118) (width 0.2) (layer "F.Cu") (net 4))
 (segment (start 168.078723 112.996673) (end 168.078723 115.580662) (width 0.2) (layer "F.Cu") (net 4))
 (segment (start 148.2 108.8) (end 132.065 124.935) (width 0.2) (layer "F.Cu") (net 4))
 (segment (start 160.886 107.699) (end 162.78105 107.699) (width 0.2) (layer "F.Cu") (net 4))
 (segment (start 175.7275 116.699999) (end 175.7275 116.5) (width 0.2) (layer "F.Cu") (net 4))
 (segment (start 159.785 108.8) (end 148.2 108.8) (width 0.2) (layer "F.Cu") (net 4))
 (segment (start 162.78105 107.699) (end 168.078723 112.996673) (width 0.2) (layer "F.Cu") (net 4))
 (segment (start 174.427499 118) (end 175.7275 116.699999) (width 0.2) (layer "F.Cu") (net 4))
 (segment (start 170.498061 118) (end 174.427499 118) (width 0.2) (layer "F.Cu") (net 4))
 (segment (start 159.785 108.8) (end 160.886 107.699) (width 0.2) (layer "F.Cu") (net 4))
 (segment (start 122.386 124.311) (end 130.626 124.311) (width 0.2) (layer "B.Cu") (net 4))
 (segment (start 130.626 124.311) (end 132.065 125.75) (width 0.2) (layer "B.Cu") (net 4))
 (segment (start 121.285 123.21) (end 122.386 124.311) (width 0.2) (layer "B.Cu") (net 4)))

